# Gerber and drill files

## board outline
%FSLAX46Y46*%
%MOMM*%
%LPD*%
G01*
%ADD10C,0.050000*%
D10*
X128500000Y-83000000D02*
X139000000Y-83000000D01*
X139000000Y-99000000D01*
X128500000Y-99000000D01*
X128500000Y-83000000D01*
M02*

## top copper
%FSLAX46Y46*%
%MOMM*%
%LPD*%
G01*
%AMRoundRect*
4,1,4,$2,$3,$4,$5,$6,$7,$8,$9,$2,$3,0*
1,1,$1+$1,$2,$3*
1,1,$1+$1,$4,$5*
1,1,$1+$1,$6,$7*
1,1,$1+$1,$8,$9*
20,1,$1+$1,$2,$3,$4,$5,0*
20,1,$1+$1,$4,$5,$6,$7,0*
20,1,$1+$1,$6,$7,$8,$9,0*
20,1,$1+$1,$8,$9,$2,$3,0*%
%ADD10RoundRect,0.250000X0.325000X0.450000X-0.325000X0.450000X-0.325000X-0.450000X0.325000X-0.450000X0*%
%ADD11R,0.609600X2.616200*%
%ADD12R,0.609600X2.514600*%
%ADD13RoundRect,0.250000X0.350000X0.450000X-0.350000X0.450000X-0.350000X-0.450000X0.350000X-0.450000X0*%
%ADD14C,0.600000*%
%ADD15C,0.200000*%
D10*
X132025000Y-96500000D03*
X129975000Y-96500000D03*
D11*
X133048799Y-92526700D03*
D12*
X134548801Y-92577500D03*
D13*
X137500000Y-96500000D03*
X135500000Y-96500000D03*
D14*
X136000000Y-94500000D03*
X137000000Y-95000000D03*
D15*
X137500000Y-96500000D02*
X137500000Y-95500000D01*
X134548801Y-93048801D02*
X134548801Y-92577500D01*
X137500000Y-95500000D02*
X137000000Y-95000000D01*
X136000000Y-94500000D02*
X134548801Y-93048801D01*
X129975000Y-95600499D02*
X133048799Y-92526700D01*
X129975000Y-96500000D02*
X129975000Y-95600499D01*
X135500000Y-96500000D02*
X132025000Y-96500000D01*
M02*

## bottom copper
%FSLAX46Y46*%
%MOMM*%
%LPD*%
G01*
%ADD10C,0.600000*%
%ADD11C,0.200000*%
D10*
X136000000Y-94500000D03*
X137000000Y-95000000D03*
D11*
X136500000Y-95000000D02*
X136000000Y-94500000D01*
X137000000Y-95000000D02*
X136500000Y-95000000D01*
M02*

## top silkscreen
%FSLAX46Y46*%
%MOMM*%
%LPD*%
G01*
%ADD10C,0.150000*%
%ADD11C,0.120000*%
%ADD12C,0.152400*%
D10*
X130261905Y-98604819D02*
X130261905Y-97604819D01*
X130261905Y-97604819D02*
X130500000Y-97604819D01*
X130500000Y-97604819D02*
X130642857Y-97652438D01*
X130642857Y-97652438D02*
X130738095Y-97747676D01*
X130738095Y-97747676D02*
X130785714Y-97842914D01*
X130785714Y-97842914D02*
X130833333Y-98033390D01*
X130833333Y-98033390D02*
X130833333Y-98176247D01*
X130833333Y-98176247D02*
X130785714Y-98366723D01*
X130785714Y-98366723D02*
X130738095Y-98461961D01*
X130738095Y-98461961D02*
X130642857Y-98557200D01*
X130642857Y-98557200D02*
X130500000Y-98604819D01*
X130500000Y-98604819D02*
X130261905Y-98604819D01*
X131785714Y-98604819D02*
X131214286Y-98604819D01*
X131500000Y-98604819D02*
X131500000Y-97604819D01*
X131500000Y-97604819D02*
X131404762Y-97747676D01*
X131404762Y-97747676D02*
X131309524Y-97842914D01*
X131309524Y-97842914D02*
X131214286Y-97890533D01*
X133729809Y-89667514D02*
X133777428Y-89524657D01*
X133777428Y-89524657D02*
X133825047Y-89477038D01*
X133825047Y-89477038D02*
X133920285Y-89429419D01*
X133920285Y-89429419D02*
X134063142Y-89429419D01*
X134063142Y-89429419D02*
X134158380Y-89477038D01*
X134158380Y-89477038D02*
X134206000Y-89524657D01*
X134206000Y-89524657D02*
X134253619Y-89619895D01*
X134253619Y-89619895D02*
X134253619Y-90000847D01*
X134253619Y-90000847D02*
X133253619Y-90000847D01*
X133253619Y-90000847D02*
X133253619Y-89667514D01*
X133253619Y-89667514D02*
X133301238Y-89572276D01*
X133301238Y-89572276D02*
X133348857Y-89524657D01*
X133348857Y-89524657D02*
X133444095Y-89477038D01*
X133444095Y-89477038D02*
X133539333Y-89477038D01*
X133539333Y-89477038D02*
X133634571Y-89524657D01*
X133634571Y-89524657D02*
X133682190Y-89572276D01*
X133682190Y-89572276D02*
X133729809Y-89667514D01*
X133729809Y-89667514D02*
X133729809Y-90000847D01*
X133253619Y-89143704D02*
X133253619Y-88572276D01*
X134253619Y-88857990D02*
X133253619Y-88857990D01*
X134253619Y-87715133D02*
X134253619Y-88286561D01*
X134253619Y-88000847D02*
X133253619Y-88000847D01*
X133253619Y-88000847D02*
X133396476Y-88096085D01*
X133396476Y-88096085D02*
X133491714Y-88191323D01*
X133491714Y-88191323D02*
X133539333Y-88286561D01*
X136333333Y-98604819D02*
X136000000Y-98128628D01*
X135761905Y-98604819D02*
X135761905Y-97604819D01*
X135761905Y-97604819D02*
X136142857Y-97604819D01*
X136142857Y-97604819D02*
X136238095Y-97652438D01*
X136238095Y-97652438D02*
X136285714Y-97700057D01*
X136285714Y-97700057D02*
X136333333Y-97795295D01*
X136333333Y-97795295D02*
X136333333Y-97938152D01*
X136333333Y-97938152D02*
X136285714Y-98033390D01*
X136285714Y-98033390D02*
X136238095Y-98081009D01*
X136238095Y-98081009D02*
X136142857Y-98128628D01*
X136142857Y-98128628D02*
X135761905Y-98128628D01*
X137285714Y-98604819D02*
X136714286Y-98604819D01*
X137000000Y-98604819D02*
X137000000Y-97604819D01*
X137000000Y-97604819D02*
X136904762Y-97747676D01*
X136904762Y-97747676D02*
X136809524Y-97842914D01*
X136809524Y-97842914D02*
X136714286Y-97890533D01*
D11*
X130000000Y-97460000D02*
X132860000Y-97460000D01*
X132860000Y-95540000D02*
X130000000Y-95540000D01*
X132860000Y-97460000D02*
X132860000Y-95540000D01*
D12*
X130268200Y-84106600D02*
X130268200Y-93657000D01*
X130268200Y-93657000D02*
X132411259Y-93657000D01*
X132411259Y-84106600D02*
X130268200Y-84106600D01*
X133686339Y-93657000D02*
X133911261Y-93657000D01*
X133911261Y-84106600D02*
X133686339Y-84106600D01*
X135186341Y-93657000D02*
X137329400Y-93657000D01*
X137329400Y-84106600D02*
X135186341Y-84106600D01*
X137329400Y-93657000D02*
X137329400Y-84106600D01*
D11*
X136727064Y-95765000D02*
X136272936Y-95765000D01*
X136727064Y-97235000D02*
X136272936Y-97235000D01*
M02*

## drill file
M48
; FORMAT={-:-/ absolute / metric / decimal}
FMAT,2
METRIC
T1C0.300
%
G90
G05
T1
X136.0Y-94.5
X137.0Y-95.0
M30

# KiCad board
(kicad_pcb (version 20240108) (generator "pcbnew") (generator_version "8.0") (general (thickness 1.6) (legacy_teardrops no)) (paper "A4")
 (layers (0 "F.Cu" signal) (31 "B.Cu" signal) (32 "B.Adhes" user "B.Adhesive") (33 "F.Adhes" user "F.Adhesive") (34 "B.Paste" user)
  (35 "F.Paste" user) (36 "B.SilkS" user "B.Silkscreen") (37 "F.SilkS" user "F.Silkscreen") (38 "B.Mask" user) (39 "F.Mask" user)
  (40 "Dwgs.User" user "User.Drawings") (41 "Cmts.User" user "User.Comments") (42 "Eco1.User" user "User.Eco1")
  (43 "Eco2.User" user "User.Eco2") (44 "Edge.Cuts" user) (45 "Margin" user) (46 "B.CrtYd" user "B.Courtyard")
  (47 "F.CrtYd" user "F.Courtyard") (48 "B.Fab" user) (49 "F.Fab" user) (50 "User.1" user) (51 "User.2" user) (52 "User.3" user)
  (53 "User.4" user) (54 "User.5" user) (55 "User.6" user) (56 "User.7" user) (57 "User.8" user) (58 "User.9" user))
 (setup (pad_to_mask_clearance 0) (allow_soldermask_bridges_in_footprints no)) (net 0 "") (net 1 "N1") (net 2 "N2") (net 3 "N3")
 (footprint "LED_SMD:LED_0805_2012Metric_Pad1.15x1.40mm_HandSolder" (layer "F.Cu") (at 131 96.5 180)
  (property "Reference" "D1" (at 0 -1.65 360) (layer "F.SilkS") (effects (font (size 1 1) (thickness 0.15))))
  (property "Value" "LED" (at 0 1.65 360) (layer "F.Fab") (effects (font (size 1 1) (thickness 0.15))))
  (fp_line (start 1 -0.96) (end -1.86 -0.96) (stroke (width 0.12) (type solid)) (layer "F.SilkS"))
  (fp_line (start -1.86 0.96) (end 1 0.96) (stroke (width 0.12) (type solid)) (layer "F.SilkS"))
  (fp_line (start -1.86 -0.96) (end -1.86 0.96) (stroke (width 0.12) (type solid)) (layer "F.SilkS"))
  (pad "1" smd roundrect (at -1.025 0 180) (size 1.15 1.4) (layers "F.Cu" "F.Paste" "F.Mask") (roundrect_rratio 0.217391) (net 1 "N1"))
  (pad "2" smd roundrect (at 1.025 0 180) (size 1.15 1.4) (layers "F.Cu" "F.Paste" "F.Mask") (roundrect_rratio 0.217391) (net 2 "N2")))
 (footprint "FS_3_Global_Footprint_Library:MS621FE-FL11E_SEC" (layer "F.Cu") (at 133.7988 88.8818 90)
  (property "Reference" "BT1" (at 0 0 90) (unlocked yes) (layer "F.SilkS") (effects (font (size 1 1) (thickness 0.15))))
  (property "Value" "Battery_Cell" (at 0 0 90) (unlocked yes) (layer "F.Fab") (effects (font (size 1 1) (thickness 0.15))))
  (fp_line (start 4.7752 -3.5306) (end -4.7752 -3.5306) (stroke (width 0.1524) (type solid)) (layer "F.SilkS"))
  (fp_line (start -4.7752 -3.5306) (end -4.7752 -1.387541) (stroke (width 0.1524) (type solid)) (layer "F.SilkS"))
  (fp_line (start 4.7752 -1.387541) (end 4.7752 -3.5306) (stroke (width 0.1524) (type solid)) (layer "F.SilkS"))
  (fp_line (start -4.7752 -0.112461) (end -4.7752 0.112461) (stroke (width 0.1524) (type solid)) (layer "F.SilkS"))
  (fp_line (start 4.7752 0.112461) (end 4.7752 -0.112461) (stroke (width 0.1524) (type solid)) (layer "F.SilkS"))
  (fp_line (start -4.7752 1.387541) (end -4.7752 3.5306) (stroke (width 0.1524) (type solid)) (layer "F.SilkS"))
  (fp_line (start 4.7752 3.5306) (end 4.7752 1.387541) (stroke (width 0.1524) (type solid)) (layer "F.SilkS"))
  (fp_line (start -4.7752 3.5306) (end 4.7752 3.5306) (stroke (width 0.1524) (type solid)) (layer "F.SilkS"))
  (pad "1" smd rect (at -3.6449 -0.750001 90) (size 2.6162 0.6096) (layers "F.Cu" "F.Paste" "F.Mask") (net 2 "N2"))
  (pad "2" smd rect (at -3.6957 0.750001 90) (size 2.5146 0.6096) (layers "F.Cu" "F.Paste" "F.Mask") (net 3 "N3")))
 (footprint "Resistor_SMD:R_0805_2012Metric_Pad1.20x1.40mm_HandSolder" (layer "F.Cu") (at 136.5 96.5 180)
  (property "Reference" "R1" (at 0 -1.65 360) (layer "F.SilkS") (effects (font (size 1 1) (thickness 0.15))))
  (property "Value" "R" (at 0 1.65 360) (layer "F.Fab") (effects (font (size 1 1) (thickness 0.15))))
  (fp_line (start -0.227064 0.735) (end 0.227064 0.735) (stroke (width 0.12) (type solid)) (layer "F.SilkS"))
  (fp_line (start -0.227064 -0.735) (end 0.227064 -0.735) (stroke (width 0.12) (type solid)) (layer "F.SilkS"))
  (pad "1" smd roundrect (at -1 0 180) (size 1.2 1.4) (layers "F.Cu" "F.Paste" "F.Mask") (roundrect_rratio 0.208333) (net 1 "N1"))
  (pad "2" smd roundrect (at 1 0 180) (size 1.2 1.4) (layers "F.Cu" "F.Paste" "F.Mask") (roundrect_rratio 0.208333) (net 3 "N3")))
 (gr_rect (start 128.5 83) (end 139 99) (stroke (width 0.05) (type default)) (fill none) (layer "Edge.Cuts"))
 (segment (start 137.5 96.5) (end 137.5 95.5) (width 0.2) (layer "F.Cu") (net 3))
 (segment (start 134.548801 93.048801) (end 134.548801 92.5775) (width 0.2) (layer "F.Cu") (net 3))
 (segment (start 137.5 95.5) (end 137 95) (width 0.2) (layer "F.Cu") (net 3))
 (segment (start 136 94.5) (end 134.548801 93.048801) (width 0.2) (layer "F.Cu") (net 3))
 (via (at 136 94.5) (size 0.6) (drill 0.3) (layers "F.Cu" "B.Cu") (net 3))
 (via (at 137 95) (size 0.6) (drill 0.3) (layers "F.Cu" "B.Cu") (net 3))
 (segment (start 136.5 95) (end 136 94.5) (width 0.2) (layer "B.Cu") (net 3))
 (segment (start 137 95) (end 136.5 95) (width 0.2) (layer "B.Cu") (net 3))
 (segment (start 129.975 95.600499) (end 133.048799 92.5267) (width 0.2) (layer "F.Cu") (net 2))
 (segment (start 129.975 96.5) (end 129.975 95.600499) (width 0.2) (layer "F.Cu") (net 2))
 (segment (start 135.5 96.5) (end 132.025 96.5) (width 0.2) (layer "F.Cu") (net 1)))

